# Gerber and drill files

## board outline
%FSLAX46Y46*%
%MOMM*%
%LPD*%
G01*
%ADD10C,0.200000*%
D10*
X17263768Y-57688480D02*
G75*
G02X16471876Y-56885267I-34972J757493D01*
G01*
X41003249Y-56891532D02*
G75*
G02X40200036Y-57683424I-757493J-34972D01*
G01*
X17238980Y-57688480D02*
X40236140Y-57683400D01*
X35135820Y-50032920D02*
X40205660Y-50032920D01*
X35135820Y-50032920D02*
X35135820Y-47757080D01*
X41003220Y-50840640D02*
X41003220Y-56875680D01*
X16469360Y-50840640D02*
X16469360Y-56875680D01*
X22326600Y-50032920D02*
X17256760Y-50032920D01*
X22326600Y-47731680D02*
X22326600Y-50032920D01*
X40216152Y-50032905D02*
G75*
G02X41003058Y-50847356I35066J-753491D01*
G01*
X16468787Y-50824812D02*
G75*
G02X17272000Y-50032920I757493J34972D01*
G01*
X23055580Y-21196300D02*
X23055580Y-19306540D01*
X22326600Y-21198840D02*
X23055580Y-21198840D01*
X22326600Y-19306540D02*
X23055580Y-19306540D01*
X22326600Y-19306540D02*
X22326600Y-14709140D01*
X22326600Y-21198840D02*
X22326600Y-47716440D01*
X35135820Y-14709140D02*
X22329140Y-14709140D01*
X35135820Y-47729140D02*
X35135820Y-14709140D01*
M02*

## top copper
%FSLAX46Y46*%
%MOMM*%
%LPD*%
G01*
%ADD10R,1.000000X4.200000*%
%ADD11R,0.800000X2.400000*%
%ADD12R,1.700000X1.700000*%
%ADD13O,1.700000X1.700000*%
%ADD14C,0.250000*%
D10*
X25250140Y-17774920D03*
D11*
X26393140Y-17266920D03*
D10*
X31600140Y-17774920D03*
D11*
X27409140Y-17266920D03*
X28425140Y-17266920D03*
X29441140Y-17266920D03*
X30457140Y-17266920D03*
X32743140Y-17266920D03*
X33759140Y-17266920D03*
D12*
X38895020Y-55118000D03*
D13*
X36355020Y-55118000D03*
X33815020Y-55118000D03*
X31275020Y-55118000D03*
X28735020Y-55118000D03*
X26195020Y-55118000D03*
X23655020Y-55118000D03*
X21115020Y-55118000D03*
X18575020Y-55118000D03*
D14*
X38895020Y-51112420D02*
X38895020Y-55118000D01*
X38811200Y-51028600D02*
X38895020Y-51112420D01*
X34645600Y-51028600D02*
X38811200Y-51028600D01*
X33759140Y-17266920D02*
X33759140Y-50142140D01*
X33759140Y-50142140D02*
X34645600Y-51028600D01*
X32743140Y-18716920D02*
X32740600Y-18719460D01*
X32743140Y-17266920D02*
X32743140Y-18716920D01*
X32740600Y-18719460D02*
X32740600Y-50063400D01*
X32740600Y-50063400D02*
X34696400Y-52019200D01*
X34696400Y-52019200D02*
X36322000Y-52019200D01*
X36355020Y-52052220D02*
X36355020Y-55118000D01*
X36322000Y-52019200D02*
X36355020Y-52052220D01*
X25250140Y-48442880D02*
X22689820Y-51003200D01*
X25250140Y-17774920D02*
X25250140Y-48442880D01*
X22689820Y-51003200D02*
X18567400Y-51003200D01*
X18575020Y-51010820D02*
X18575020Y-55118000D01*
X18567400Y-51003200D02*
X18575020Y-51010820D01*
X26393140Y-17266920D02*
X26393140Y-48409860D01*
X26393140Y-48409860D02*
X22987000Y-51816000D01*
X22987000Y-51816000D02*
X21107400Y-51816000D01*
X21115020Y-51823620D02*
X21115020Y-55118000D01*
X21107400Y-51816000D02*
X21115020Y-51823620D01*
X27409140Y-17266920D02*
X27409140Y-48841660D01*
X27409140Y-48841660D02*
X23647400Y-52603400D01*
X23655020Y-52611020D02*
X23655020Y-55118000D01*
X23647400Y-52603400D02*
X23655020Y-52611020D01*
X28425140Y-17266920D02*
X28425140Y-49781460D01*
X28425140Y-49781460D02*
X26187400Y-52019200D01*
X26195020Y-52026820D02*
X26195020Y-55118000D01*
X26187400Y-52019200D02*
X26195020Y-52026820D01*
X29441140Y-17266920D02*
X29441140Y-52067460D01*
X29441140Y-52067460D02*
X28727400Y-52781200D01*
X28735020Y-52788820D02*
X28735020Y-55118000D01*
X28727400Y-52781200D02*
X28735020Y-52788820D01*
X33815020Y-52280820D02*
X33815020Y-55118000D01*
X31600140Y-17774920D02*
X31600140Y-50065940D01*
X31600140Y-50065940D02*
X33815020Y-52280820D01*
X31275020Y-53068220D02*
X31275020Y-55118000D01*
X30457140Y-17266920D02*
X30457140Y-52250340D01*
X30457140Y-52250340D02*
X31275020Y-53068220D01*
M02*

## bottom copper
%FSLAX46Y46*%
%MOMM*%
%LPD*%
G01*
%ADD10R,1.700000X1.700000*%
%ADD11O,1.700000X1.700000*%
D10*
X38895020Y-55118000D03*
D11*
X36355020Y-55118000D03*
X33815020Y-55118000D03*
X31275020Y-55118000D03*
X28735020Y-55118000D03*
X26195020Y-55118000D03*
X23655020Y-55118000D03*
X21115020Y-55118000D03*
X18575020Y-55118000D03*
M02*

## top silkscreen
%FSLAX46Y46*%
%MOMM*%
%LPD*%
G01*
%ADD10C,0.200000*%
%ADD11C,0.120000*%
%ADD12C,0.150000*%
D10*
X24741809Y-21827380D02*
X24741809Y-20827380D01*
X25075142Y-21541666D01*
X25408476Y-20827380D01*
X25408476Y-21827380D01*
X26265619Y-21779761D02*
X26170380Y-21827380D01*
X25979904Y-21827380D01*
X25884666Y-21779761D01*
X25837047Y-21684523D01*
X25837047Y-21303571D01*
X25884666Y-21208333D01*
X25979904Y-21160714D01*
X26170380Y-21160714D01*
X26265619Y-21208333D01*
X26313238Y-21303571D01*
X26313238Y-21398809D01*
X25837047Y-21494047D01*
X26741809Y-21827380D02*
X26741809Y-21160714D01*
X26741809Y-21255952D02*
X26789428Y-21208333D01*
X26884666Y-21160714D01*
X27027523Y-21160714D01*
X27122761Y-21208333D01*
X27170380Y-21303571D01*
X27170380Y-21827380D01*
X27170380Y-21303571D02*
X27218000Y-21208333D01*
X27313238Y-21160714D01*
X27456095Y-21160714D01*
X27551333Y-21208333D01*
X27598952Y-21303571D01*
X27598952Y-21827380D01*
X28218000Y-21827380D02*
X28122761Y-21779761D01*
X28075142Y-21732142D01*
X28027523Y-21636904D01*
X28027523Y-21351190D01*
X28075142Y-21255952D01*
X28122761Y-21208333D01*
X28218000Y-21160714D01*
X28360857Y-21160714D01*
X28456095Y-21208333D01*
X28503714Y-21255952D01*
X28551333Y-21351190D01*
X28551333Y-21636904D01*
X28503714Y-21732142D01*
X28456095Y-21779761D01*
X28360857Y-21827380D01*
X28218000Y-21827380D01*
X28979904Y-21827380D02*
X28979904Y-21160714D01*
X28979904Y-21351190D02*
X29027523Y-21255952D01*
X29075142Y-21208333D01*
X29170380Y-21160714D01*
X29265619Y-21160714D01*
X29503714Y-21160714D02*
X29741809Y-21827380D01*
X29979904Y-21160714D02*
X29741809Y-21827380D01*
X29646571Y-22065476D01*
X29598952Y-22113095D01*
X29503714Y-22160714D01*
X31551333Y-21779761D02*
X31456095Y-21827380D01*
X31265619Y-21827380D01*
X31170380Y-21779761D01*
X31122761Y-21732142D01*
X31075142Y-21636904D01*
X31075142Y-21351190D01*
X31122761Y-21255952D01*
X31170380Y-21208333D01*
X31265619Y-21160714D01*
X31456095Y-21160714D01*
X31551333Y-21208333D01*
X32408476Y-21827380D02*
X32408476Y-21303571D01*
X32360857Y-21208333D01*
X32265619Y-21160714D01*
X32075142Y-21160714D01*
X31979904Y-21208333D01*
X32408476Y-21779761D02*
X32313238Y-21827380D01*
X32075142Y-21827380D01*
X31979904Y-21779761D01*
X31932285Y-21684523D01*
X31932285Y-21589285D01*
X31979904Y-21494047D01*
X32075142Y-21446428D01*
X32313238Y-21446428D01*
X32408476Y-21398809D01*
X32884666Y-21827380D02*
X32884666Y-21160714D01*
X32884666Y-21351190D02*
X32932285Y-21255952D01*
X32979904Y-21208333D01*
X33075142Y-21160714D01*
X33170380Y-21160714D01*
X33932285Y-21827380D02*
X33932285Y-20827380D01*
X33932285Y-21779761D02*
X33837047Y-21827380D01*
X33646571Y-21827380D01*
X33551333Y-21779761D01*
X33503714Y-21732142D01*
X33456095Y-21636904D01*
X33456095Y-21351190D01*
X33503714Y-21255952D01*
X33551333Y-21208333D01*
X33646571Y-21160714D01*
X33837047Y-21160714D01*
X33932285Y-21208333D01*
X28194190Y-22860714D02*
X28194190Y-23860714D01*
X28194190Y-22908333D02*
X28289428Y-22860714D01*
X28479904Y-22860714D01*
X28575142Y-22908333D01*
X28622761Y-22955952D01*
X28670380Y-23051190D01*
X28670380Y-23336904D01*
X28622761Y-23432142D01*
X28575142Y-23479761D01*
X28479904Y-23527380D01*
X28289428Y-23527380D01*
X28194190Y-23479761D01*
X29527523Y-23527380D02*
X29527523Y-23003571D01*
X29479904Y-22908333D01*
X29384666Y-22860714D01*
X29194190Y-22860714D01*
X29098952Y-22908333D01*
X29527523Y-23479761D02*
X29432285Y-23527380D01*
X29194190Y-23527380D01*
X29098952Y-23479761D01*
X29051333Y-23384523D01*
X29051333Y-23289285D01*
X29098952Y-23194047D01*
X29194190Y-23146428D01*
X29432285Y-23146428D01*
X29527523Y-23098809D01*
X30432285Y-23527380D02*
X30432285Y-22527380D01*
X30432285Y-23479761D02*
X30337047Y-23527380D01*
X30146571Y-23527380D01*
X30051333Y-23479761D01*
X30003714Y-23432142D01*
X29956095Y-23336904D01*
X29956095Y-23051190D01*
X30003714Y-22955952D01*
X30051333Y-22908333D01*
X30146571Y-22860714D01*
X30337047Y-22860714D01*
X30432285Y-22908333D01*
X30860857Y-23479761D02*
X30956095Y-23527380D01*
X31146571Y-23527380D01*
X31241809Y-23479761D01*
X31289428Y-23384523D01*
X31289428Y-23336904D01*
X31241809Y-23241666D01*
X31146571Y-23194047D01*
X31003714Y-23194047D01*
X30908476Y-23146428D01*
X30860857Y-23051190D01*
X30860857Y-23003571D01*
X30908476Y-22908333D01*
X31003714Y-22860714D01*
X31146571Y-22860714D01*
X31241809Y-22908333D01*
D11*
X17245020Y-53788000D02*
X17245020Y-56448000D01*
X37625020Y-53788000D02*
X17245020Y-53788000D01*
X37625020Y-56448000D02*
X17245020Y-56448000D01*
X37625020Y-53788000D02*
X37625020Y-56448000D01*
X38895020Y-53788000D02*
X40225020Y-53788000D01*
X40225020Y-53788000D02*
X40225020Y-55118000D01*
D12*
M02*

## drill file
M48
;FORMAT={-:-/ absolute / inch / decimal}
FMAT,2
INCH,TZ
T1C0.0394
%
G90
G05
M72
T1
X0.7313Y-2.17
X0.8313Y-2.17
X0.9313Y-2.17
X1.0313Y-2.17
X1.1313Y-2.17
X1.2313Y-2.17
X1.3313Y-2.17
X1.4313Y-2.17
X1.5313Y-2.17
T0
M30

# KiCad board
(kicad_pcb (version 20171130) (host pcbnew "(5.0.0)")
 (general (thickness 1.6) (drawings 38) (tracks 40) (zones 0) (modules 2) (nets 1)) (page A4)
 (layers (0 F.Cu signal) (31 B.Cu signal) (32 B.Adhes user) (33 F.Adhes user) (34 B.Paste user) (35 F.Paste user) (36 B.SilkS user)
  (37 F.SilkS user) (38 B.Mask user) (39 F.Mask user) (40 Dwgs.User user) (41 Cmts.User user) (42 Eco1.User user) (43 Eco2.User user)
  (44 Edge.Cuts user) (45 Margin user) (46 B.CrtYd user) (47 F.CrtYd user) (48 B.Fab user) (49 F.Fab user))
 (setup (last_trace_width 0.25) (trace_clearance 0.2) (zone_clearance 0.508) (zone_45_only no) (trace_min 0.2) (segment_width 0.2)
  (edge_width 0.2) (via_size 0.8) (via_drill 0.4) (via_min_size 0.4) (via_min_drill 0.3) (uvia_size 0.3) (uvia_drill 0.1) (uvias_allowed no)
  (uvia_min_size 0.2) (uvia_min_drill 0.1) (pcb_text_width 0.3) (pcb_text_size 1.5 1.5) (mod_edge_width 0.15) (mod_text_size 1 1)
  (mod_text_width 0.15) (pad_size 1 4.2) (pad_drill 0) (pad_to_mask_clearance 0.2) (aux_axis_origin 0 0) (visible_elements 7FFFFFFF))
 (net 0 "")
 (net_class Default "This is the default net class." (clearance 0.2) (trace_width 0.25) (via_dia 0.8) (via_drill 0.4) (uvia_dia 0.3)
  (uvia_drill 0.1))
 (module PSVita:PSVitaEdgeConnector (layer F.Cu) (at 30.33014 17.26692)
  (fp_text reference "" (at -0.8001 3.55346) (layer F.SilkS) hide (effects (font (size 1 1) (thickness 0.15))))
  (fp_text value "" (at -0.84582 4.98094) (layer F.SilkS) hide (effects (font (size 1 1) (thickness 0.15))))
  (pad 9 smd rect (at -5.08 0.508) (size 1 4.2) (layers F.Cu F.Paste F.Mask))
  (pad 8 smd rect (at -3.937 0) (size 0.8 2.4) (layers F.Cu F.Paste F.Mask))
  (pad 3 smd rect (at 1.27 0.508) (size 1 4.2) (layers F.Cu F.Paste F.Mask))
  (pad 7 smd rect (at -2.921 0) (size 0.8 2.4) (layers F.Cu F.Paste F.Mask))
  (pad 6 smd rect (at -1.905 0) (size 0.8 2.4) (layers F.Cu F.Paste F.Mask))
  (pad 5 smd rect (at -0.889 0) (size 0.8 2.4) (layers F.Cu F.Paste F.Mask))
  (pad 4 smd rect (at 0.127 0) (size 0.8 2.4) (layers F.Cu F.Paste F.Mask))
  (pad 2 smd rect (at 2.413 0) (size 0.8 2.4) (layers F.Cu F.Paste F.Mask))
  (pad 1 smd rect (at 3.429 0) (size 0.8 2.4) (layers F.Cu F.Paste F.Mask)))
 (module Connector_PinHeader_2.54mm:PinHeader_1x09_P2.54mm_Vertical (layer F.Cu) (at 38.89502 55.118 270)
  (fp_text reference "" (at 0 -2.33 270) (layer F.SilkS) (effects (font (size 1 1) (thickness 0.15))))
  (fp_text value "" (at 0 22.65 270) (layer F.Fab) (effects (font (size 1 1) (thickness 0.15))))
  (fp_line (start -1.33 21.65) (end 1.33 21.65) (layer F.SilkS) (width 0.12))
  (fp_line (start -1.33 1.27) (end -1.33 21.65) (layer F.SilkS) (width 0.12))
  (fp_line (start 1.33 1.27) (end 1.33 21.65) (layer F.SilkS) (width 0.12))
  (fp_line (start -1.33 1.27) (end 1.33 1.27) (layer F.SilkS) (width 0.12))
  (fp_line (start -1.33 0) (end -1.33 -1.33) (layer F.SilkS) (width 0.12))
  (fp_line (start -1.33 -1.33) (end 0 -1.33) (layer F.SilkS) (width 0.12))
  (pad 1 thru_hole rect (at 0 0 270) (size 1.7 1.7) (drill 1) (layers *.Cu *.Mask))
  (pad 2 thru_hole oval (at 0 2.54 270) (size 1.7 1.7) (drill 1) (layers *.Cu *.Mask))
  (pad 3 thru_hole oval (at 0 5.08 270) (size 1.7 1.7) (drill 1) (layers *.Cu *.Mask))
  (pad 4 thru_hole oval (at 0 7.62 270) (size 1.7 1.7) (drill 1) (layers *.Cu *.Mask))
  (pad 5 thru_hole oval (at 0 10.16 270) (size 1.7 1.7) (drill 1) (layers *.Cu *.Mask))
  (pad 6 thru_hole oval (at 0 12.7 270) (size 1.7 1.7) (drill 1) (layers *.Cu *.Mask))
  (pad 7 thru_hole oval (at 0 15.24 270) (size 1.7 1.7) (drill 1) (layers *.Cu *.Mask))
  (pad 8 thru_hole oval (at 0 17.78 270) (size 1.7 1.7) (drill 1) (layers *.Cu *.Mask))
  (pad 9 thru_hole oval (at 0 20.32 270) (size 1.7 1.7) (drill 1) (layers *.Cu *.Mask)))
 (gr_arc (start 17.228796 56.930987) (end 16.471876 56.885267) (angle -96.1) (layer Edge.Cuts) (width 0.2))
 (gr_arc (start 40.245756 56.926504) (end 40.200036 57.683424) (angle -96.1) (layer Edge.Cuts) (width 0.2))
 (gr_line (start 17.23898 57.68848) (end 40.23614 57.6834) (layer Edge.Cuts) (width 0.2))
 (gr_line (start 35.13582 50.03292) (end 40.20566 50.03292) (layer Edge.Cuts) (width 0.2))
 (gr_line (start 35.13582 50.03292) (end 35.13582 47.75708) (layer Edge.Cuts) (width 0.2))
 (gr_line (start 41.00322 50.84064) (end 41.00322 56.87568) (layer Edge.Cuts) (width 0.2))
 (gr_line (start 16.46936 50.84064) (end 16.46936 56.87568) (layer Edge.Cuts) (width 0.2))
 (gr_line (start 22.3266 50.03292) (end 17.25676 50.03292) (layer Edge.Cuts) (width 0.2))
 (gr_line (start 22.3266 47.73168) (end 22.3266 50.03292) (layer Edge.Cuts) (width 0.2))
 (gr_arc (start 40.251218 50.786396) (end 41.003058 50.847356) (angle -97.3) (layer Edge.Cuts) (width 0.2))
 (gr_arc (start 17.22628 50.78984) (end 17.272 50.03292) (angle -96.1) (layer Edge.Cuts) (width 0.2))
 (gr_line (start 23.05558 21.1963) (end 23.05558 19.30654) (layer Edge.Cuts) (width 0.2))
 (gr_line (start 22.3266 21.19884) (end 23.05558 21.19884) (layer Edge.Cuts) (width 0.2))
 (gr_line (start 22.3266 19.30654) (end 23.05558 19.30654) (layer Edge.Cuts) (width 0.2))
 (gr_line (start 22.3266 19.30654) (end 22.3266 14.70914) (layer Edge.Cuts) (width 0.2))
 (gr_line (start 22.3266 21.19884) (end 22.3266 47.71644) (layer Edge.Cuts) (width 0.2))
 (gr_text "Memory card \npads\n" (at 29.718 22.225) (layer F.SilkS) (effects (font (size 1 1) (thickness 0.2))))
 (gr_line (start 35.13582 14.70914) (end 22.32914 14.70914) (layer Edge.Cuts) (width 0.2))
 (gr_line (start 35.13582 47.72914) (end 35.13582 14.70914) (layer Edge.Cuts) (width 0.2))
 (segment (start 38.89502 51.11242) (end 38.89502 55.118) (width 0.25) (layer F.Cu) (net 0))
 (segment (start 38.8112 51.0286) (end 38.89502 51.11242) (width 0.25) (layer F.Cu) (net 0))
 (segment (start 34.6456 51.0286) (end 38.8112 51.0286) (width 0.25) (layer F.Cu) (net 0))
 (segment (start 33.75914 17.26692) (end 33.75914 50.14214) (width 0.25) (layer F.Cu) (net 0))
 (segment (start 33.75914 50.14214) (end 34.6456 51.0286) (width 0.25) (layer F.Cu) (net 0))
 (segment (start 32.74314 18.71692) (end 32.7406 18.71946) (width 0.25) (layer F.Cu) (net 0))
 (segment (start 32.74314 17.26692) (end 32.74314 18.71692) (width 0.25) (layer F.Cu) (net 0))
 (segment (start 32.7406 18.71946) (end 32.7406 50.0634) (width 0.25) (layer F.Cu) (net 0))
 (segment (start 32.7406 50.0634) (end 34.6964 52.0192) (width 0.25) (layer F.Cu) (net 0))
 (segment (start 34.6964 52.0192) (end 36.322 52.0192) (width 0.25) (layer F.Cu) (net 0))
 (segment (start 36.35502 52.05222) (end 36.35502 55.118) (width 0.25) (layer F.Cu) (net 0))
 (segment (start 36.322 52.0192) (end 36.35502 52.05222) (width 0.25) (layer F.Cu) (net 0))
 (segment (start 25.25014 48.44288) (end 22.68982 51.0032) (width 0.25) (layer F.Cu) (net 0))
 (segment (start 25.25014 17.77492) (end 25.25014 48.44288) (width 0.25) (layer F.Cu) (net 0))
 (segment (start 22.68982 51.0032) (end 18.5674 51.0032) (width 0.25) (layer F.Cu) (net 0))
 (segment (start 18.57502 51.01082) (end 18.57502 55.118) (width 0.25) (layer F.Cu) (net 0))
 (segment (start 18.5674 51.0032) (end 18.57502 51.01082) (width 0.25) (layer F.Cu) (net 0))
 (segment (start 26.39314 17.26692) (end 26.39314 48.40986) (width 0.25) (layer F.Cu) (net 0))
 (segment (start 26.39314 48.40986) (end 22.987 51.816) (width 0.25) (layer F.Cu) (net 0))
 (segment (start 22.987 51.816) (end 21.1074 51.816) (width 0.25) (layer F.Cu) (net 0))
 (segment (start 21.11502 51.82362) (end 21.11502 55.118) (width 0.25) (layer F.Cu) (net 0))
 (segment (start 21.1074 51.816) (end 21.11502 51.82362) (width 0.25) (layer F.Cu) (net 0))
 (segment (start 27.40914 17.26692) (end 27.40914 48.84166) (width 0.25) (layer F.Cu) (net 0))
 (segment (start 27.40914 48.84166) (end 23.6474 52.6034) (width 0.25) (layer F.Cu) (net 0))
 (segment (start 23.65502 52.61102) (end 23.65502 55.118) (width 0.25) (layer F.Cu) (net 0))
 (segment (start 23.6474 52.6034) (end 23.65502 52.61102) (width 0.25) (layer F.Cu) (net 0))
 (segment (start 28.42514 17.26692) (end 28.42514 49.78146) (width 0.25) (layer F.Cu) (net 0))
 (segment (start 28.42514 49.78146) (end 26.1874 52.0192) (width 0.25) (layer F.Cu) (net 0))
 (segment (start 26.19502 52.02682) (end 26.19502 55.118) (width 0.25) (layer F.Cu) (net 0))
 (segment (start 26.1874 52.0192) (end 26.19502 52.02682) (width 0.25) (layer F.Cu) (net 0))
 (segment (start 29.44114 17.26692) (end 29.44114 52.06746) (width 0.25) (layer F.Cu) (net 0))
 (segment (start 29.44114 52.06746) (end 28.7274 52.7812) (width 0.25) (layer F.Cu) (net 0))
 (segment (start 28.73502 52.78882) (end 28.73502 55.118) (width 0.25) (layer F.Cu) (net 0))
 (segment (start 28.7274 52.7812) (end 28.73502 52.78882) (width 0.25) (layer F.Cu) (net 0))
 (segment (start 33.81502 52.28082) (end 33.81502 55.118) (width 0.25) (layer F.Cu) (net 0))
 (segment (start 31.60014 17.77492) (end 31.60014 50.06594) (width 0.25) (layer F.Cu) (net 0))
 (segment (start 31.60014 50.06594) (end 33.81502 52.28082) (width 0.25) (layer F.Cu) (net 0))
 (segment (start 31.27502 53.06822) (end 31.27502 55.118) (width 0.25) (layer F.Cu) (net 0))
 (segment (start 30.45714 17.26692) (end 30.45714 52.25034) (width 0.25) (layer F.Cu) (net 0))
 (segment (start 30.45714 52.25034) (end 31.27502 53.06822) (width 0.25) (layer F.Cu) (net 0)))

